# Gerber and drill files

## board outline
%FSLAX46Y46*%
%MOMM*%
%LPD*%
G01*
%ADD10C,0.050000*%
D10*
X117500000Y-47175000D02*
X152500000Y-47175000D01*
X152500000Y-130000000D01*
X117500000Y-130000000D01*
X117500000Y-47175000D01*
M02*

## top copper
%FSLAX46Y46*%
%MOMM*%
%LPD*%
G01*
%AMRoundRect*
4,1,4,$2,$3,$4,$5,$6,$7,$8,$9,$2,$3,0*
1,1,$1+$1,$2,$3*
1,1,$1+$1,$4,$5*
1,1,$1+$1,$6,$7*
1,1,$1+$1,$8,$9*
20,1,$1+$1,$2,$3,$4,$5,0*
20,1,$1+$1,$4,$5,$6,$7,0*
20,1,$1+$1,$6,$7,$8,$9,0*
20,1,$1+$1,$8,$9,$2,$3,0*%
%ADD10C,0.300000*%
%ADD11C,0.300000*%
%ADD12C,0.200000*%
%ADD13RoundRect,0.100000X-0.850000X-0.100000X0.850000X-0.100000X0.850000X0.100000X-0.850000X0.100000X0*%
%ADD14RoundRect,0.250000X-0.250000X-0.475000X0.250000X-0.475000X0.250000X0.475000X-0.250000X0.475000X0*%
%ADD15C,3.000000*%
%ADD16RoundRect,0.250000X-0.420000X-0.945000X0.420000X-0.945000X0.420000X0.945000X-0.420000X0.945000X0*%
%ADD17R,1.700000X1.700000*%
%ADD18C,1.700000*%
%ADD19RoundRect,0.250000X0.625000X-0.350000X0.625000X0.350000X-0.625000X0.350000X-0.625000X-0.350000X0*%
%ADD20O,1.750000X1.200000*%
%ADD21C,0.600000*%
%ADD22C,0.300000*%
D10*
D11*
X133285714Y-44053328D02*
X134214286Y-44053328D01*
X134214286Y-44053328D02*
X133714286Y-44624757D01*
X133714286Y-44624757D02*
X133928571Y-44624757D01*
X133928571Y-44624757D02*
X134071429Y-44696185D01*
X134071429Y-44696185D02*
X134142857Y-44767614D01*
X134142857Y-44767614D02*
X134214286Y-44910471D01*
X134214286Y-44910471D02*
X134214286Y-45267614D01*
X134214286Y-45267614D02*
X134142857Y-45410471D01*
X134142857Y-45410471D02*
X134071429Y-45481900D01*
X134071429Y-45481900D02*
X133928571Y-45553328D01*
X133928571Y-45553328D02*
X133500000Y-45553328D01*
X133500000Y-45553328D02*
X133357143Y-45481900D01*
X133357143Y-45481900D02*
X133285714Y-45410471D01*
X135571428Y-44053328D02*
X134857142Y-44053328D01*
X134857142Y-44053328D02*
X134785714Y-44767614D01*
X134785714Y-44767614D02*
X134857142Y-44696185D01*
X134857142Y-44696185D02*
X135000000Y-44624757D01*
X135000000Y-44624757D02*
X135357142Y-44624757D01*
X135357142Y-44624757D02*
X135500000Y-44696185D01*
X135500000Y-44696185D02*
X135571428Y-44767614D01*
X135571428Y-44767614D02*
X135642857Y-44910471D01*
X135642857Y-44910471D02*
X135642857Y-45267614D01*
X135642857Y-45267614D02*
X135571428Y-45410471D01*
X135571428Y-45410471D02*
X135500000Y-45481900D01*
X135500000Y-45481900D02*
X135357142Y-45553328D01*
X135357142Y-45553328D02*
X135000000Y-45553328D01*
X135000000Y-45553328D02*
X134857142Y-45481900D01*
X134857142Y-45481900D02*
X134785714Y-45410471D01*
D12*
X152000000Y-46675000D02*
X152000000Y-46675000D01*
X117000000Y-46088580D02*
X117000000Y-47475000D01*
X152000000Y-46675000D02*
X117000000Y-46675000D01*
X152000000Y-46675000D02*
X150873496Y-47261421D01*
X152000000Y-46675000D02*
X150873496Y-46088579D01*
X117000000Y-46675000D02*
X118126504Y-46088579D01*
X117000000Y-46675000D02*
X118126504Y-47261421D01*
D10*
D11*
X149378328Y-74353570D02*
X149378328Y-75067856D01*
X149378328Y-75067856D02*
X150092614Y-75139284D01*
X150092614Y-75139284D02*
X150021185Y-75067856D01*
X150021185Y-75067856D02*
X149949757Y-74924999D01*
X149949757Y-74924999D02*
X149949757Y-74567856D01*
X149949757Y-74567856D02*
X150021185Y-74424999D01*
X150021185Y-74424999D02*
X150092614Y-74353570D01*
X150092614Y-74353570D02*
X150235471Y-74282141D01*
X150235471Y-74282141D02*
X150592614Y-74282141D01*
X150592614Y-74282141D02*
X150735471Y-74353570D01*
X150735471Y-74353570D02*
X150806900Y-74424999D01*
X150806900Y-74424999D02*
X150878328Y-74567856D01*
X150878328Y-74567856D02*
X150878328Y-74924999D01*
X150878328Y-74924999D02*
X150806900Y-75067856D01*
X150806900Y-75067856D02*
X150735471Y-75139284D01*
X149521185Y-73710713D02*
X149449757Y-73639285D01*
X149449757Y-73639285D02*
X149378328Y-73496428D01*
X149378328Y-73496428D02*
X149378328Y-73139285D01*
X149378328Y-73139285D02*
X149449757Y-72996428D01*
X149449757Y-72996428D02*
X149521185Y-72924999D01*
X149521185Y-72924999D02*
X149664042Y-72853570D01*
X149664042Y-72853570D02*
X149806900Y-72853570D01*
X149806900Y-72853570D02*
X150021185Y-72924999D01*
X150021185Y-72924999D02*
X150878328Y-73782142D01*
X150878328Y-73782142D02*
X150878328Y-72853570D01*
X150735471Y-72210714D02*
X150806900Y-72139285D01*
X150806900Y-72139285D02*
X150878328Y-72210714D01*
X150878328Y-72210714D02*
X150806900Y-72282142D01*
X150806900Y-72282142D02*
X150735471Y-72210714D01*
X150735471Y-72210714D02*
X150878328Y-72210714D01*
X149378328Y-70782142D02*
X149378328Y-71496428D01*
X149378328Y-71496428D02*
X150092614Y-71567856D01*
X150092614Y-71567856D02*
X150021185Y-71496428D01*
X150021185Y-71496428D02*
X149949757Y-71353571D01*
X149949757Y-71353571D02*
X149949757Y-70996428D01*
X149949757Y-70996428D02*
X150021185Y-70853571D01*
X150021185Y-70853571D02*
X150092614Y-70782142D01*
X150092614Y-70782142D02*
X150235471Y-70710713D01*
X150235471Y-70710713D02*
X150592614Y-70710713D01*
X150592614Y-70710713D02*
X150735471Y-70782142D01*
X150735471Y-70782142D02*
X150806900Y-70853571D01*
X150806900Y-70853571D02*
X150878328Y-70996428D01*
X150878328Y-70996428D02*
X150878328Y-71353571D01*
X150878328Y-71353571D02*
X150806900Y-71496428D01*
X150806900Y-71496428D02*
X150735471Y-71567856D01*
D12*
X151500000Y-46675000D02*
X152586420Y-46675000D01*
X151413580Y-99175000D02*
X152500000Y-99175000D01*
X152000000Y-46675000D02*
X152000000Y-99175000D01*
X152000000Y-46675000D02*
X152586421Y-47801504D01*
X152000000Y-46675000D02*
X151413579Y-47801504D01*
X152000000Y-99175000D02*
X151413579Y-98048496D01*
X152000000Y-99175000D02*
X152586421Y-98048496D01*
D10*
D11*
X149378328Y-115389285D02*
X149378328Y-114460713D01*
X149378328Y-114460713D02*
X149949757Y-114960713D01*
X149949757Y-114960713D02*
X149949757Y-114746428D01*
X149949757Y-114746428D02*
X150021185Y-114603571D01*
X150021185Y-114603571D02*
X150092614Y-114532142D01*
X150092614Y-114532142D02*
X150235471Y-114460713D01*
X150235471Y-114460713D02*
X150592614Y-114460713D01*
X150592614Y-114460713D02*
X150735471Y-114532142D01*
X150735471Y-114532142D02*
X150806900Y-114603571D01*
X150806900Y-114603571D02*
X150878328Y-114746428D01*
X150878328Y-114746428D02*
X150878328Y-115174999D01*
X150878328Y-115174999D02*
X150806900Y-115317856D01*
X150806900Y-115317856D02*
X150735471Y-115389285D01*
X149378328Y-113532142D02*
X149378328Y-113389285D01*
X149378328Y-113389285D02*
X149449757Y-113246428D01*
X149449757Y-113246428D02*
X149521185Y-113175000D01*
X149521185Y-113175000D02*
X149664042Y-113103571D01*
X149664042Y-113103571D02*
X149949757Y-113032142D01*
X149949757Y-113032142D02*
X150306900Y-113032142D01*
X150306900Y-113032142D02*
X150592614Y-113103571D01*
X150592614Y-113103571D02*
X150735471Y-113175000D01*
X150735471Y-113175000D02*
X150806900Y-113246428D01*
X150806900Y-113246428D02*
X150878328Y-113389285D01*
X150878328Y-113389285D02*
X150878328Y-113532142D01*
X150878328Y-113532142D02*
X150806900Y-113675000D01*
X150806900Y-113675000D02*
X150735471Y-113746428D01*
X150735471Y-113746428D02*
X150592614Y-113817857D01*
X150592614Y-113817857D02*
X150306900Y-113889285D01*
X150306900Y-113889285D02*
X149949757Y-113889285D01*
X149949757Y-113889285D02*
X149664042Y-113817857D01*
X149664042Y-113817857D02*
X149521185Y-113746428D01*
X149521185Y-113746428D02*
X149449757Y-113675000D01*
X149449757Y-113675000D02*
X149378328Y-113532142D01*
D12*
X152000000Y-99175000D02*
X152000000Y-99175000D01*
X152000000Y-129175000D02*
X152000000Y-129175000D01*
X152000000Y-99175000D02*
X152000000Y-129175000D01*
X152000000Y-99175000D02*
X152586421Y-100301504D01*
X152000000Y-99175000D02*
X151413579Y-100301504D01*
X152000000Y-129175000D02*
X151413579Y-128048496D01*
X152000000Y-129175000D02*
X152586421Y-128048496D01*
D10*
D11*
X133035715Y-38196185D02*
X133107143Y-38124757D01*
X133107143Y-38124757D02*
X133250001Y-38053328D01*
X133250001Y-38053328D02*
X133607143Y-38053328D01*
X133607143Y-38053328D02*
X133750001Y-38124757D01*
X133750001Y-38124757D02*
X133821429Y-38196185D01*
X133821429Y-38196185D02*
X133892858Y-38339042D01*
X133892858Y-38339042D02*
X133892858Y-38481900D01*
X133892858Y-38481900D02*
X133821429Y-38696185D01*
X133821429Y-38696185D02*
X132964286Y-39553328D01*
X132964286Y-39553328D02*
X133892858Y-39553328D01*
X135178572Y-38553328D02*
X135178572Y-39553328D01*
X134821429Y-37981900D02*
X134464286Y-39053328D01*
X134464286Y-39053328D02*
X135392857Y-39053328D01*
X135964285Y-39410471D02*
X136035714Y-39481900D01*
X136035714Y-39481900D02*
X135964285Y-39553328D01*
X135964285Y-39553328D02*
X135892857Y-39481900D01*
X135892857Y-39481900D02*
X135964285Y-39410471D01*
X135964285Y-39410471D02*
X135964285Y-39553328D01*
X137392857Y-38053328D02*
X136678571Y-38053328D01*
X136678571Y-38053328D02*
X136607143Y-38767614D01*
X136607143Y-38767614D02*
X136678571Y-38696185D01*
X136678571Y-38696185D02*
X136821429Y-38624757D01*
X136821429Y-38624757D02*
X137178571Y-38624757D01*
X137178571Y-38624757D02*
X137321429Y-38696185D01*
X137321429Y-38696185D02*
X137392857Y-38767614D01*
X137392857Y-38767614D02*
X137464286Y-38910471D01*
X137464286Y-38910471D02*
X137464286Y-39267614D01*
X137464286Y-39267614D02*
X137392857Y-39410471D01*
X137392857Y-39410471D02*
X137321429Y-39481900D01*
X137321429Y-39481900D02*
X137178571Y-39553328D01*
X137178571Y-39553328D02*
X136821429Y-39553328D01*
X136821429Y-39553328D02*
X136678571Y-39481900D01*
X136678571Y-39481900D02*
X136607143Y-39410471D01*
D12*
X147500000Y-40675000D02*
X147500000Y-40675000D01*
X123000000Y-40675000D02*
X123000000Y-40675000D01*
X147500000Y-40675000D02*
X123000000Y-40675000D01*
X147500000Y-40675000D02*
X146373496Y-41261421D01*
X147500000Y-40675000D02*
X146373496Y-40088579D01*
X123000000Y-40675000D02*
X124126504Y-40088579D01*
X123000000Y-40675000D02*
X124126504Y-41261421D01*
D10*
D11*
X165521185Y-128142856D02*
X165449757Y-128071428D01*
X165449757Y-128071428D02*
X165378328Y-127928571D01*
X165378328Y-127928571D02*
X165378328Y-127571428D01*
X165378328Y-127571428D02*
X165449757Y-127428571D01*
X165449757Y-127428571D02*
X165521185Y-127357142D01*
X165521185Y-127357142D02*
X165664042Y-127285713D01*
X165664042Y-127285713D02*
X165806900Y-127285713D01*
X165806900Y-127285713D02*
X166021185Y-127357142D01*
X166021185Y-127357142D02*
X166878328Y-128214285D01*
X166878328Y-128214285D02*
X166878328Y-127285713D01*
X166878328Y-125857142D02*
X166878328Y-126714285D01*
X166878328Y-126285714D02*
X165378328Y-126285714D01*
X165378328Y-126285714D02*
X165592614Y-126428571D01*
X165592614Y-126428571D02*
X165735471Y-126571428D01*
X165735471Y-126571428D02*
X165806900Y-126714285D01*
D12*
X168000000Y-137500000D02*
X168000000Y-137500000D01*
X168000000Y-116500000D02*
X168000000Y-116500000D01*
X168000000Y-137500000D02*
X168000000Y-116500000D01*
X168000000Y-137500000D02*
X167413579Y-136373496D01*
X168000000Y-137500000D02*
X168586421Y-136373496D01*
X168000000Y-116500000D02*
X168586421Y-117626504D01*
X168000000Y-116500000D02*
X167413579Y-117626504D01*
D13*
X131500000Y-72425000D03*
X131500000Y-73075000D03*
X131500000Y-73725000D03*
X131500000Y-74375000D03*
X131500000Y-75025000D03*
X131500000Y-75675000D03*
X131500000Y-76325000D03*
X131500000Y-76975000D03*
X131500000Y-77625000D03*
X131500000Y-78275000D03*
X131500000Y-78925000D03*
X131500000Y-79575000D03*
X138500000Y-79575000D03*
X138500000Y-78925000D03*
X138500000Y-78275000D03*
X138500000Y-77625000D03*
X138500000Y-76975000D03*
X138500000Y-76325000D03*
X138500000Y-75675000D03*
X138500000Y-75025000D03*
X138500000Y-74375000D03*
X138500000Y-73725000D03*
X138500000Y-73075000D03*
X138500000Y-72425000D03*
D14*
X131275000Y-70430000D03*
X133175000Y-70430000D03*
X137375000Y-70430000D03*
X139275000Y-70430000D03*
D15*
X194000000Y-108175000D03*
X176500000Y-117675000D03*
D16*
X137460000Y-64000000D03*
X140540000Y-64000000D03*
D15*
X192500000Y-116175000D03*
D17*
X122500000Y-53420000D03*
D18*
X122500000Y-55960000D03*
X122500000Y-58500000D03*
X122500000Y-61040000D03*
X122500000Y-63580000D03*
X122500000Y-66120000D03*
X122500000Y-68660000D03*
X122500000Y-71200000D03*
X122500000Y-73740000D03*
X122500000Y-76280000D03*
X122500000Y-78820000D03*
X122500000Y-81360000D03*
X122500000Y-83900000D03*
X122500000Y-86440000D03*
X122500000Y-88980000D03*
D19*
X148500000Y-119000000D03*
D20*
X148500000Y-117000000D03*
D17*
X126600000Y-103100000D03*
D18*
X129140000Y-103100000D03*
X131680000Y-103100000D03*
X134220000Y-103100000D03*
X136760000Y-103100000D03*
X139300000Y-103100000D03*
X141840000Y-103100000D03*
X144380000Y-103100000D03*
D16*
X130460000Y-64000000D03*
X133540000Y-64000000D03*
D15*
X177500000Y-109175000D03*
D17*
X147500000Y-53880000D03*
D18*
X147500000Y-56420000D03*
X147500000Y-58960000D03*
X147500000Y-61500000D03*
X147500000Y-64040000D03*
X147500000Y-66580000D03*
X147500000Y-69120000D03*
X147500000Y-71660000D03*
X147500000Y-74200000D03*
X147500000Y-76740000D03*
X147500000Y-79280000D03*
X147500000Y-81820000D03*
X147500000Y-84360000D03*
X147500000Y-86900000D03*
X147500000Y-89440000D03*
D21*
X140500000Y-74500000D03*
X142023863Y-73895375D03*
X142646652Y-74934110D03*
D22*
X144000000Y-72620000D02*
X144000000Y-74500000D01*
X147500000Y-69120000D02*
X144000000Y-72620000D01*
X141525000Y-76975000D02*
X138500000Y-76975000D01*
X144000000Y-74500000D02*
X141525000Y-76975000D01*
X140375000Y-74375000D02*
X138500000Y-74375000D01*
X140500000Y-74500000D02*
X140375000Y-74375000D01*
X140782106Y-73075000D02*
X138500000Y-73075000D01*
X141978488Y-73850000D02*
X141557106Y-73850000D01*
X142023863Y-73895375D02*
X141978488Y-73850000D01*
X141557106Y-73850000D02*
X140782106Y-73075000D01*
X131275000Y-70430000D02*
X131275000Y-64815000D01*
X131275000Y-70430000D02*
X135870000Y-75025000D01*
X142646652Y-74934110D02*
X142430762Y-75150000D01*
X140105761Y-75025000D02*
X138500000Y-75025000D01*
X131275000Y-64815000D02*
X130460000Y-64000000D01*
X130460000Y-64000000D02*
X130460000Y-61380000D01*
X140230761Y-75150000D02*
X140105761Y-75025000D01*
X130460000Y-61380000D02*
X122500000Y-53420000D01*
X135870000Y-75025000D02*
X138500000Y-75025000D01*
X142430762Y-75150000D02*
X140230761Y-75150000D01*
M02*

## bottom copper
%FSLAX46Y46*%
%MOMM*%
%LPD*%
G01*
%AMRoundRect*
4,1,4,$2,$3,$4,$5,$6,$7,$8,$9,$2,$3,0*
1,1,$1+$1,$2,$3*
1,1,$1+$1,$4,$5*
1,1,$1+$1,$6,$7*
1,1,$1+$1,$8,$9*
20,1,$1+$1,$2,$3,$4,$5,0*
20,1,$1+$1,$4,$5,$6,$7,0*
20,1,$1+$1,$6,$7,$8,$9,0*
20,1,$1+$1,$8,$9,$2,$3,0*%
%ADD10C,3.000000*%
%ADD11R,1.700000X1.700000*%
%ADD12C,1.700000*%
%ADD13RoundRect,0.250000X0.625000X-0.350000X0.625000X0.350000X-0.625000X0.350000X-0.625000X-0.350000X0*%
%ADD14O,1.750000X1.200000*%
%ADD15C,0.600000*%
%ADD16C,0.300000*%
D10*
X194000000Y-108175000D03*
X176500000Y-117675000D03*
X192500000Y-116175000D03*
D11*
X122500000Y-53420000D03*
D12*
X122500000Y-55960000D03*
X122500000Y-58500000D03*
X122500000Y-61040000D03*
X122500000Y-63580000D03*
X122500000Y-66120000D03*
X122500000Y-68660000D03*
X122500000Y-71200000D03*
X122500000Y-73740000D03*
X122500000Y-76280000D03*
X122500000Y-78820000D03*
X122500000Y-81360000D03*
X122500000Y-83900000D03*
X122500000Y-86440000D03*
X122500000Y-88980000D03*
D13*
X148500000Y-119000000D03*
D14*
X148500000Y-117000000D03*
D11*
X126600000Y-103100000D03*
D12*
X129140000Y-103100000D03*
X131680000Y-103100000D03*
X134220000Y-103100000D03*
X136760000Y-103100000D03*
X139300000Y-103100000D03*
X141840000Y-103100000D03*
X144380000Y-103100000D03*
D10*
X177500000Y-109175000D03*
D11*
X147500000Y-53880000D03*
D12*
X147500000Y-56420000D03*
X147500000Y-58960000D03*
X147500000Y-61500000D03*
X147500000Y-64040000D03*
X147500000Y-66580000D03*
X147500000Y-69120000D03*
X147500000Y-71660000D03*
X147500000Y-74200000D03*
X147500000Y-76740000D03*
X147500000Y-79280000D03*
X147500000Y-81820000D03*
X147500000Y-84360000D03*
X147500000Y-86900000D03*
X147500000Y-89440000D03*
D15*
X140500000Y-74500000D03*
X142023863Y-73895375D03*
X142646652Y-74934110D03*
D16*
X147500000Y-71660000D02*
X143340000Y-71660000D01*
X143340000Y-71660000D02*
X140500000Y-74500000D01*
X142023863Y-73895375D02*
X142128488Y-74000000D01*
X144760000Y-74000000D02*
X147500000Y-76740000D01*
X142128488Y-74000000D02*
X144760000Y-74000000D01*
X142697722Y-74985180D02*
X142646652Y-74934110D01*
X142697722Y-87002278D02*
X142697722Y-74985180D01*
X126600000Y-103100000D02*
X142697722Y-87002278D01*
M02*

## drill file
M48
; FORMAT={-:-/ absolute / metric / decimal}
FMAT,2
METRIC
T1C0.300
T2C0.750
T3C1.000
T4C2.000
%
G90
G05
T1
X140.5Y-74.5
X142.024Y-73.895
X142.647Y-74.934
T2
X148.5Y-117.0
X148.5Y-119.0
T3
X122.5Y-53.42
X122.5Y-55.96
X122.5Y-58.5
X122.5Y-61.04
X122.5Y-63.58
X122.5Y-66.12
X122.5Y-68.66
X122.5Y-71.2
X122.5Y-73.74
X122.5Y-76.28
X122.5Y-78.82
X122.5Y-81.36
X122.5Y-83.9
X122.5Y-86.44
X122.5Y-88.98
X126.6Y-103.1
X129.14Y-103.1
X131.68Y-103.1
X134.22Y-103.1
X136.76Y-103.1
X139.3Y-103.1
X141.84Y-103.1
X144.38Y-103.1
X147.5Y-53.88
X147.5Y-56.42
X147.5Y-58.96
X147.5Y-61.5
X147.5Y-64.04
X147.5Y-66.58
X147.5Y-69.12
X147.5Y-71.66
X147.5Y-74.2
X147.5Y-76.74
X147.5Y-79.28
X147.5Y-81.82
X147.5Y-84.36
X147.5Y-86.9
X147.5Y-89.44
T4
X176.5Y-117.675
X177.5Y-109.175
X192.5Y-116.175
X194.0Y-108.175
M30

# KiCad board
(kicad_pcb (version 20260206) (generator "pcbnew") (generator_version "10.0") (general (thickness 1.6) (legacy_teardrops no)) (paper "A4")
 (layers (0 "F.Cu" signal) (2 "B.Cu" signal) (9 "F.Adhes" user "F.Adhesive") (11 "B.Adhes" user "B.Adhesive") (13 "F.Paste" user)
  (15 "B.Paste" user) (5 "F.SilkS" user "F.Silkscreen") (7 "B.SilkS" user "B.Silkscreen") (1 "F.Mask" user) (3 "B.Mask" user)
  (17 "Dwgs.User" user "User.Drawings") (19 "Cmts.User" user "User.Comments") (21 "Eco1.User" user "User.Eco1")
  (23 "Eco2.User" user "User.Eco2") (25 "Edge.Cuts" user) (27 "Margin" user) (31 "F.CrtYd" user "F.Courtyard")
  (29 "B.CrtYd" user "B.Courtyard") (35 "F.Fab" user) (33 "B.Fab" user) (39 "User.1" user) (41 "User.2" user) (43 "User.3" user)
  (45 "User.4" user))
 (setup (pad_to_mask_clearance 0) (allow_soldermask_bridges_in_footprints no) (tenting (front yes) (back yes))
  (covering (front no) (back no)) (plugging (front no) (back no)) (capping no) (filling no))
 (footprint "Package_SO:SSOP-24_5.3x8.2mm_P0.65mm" (layer "F.Cu") (at 135 76)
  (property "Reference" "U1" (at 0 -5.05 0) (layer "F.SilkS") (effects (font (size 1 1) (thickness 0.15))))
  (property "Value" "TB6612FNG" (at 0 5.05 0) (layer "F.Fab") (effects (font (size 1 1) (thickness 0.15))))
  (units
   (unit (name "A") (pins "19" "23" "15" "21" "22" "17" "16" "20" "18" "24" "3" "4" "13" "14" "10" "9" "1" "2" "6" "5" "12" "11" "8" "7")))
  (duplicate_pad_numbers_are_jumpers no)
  (pad "1" smd roundrect (at -3.5 -3.575) (size 1.9 0.4) (layers "F.Cu" "F.Mask" "F.Paste") (roundrect_rratio 0.25) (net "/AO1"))
  (pad "2" smd roundrect (at -3.5 -2.925) (size 1.9 0.4) (layers "F.Cu" "F.Mask" "F.Paste") (roundrect_rratio 0.25) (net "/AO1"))
  (pad "3" smd roundrect (at -3.5 -2.275) (size 1.9 0.4) (layers "F.Cu" "F.Mask" "F.Paste") (roundrect_rratio 0.25) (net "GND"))
  (pad "4" smd roundrect (at -3.5 -1.625) (size 1.9 0.4) (layers "F.Cu" "F.Mask" "F.Paste") (roundrect_rratio 0.25) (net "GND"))
  (pad "5" smd roundrect (at -3.5 -0.975) (size 1.9 0.4) (layers "F.Cu" "F.Mask" "F.Paste") (roundrect_rratio 0.25) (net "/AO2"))
  (pad "6" smd roundrect (at -3.5 -0.325) (size 1.9 0.4) (layers "F.Cu" "F.Mask" "F.Paste") (roundrect_rratio 0.25) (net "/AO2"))
  (pad "7" smd roundrect (at -3.5 0.325) (size 1.9 0.4) (layers "F.Cu" "F.Mask" "F.Paste") (roundrect_rratio 0.25) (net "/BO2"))
  (pad "8" smd roundrect (at -3.5 0.975) (size 1.9 0.4) (layers "F.Cu" "F.Mask" "F.Paste") (roundrect_rratio 0.25) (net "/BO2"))
  (pad "9" smd roundrect (at -3.5 1.625) (size 1.9 0.4) (layers "F.Cu" "F.Mask" "F.Paste") (roundrect_rratio 0.25) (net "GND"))
  (pad "10" smd roundrect (at -3.5 2.275) (size 1.9 0.4) (layers "F.Cu" "F.Mask" "F.Paste") (roundrect_rratio 0.25) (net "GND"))
  (pad "11" smd roundrect (at -3.5 2.925) (size 1.9 0.4) (layers "F.Cu" "F.Mask" "F.Paste") (roundrect_rratio 0.25) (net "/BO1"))
  (pad "12" smd roundrect (at -3.5 3.575) (size 1.9 0.4) (layers "F.Cu" "F.Mask" "F.Paste") (roundrect_rratio 0.25) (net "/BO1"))
  (pad "13" smd roundrect (at 3.5 3.575) (size 1.9 0.4) (layers "F.Cu" "F.Mask" "F.Paste") (roundrect_rratio 0.25) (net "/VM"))
  (pad "14" smd roundrect (at 3.5 2.925) (size 1.9 0.4) (layers "F.Cu" "F.Mask" "F.Paste") (roundrect_rratio 0.25) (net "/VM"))
  (pad "15" smd roundrect (at 3.5 2.275) (size 1.9 0.4) (layers "F.Cu" "F.Mask" "F.Paste") (roundrect_rratio 0.25) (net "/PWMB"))
  (pad "16" smd roundrect (at 3.5 1.625) (size 1.9 0.4) (layers "F.Cu" "F.Mask" "F.Paste") (roundrect_rratio 0.25) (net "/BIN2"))
  (pad "17" smd roundrect (at 3.5 0.975) (size 1.9 0.4) (layers "F.Cu" "F.Mask" "F.Paste") (roundrect_rratio 0.25) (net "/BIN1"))
  (pad "18" smd roundrect (at 3.5 0.325) (size 1.9 0.4) (layers "F.Cu" "F.Mask" "F.Paste") (roundrect_rratio 0.25) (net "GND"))
  (pad "19" smd roundrect (at 3.5 -0.325) (size 1.9 0.4) (layers "F.Cu" "F.Mask" "F.Paste") (roundrect_rratio 0.25) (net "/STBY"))
  (pad "20" smd roundrect (at 3.5 -0.975) (size 1.9 0.4) (layers "F.Cu" "F.Mask" "F.Paste") (roundrect_rratio 0.25) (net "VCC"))
  (pad "21" smd roundrect (at 3.5 -1.625) (size 1.9 0.4) (layers "F.Cu" "F.Mask" "F.Paste") (roundrect_rratio 0.25) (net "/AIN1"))
  (pad "22" smd roundrect (at 3.5 -2.275) (size 1.9 0.4) (layers "F.Cu" "F.Mask" "F.Paste") (roundrect_rratio 0.25) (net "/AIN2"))
  (pad "23" smd roundrect (at 3.5 -2.925) (size 1.9 0.4) (layers "F.Cu" "F.Mask" "F.Paste") (roundrect_rratio 0.25) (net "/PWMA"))
  (pad "24" smd roundrect (at 3.5 -3.575) (size 1.9 0.4) (layers "F.Cu" "F.Mask" "F.Paste") (roundrect_rratio 0.25) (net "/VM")))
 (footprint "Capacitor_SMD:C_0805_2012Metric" (layer "F.Cu") (at 132.225 70.43)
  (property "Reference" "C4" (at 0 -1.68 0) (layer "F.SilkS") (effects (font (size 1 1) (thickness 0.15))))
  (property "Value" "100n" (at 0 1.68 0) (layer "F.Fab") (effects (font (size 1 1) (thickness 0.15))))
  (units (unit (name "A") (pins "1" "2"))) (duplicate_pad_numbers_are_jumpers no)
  (pad "1" smd roundrect (at -0.95 0) (size 1 1.45) (layers "F.Cu" "F.Mask" "F.Paste") (roundrect_rratio 0.25) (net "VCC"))
  (pad "2" smd roundrect (at 0.95 0) (size 1 1.45) (layers "F.Cu" "F.Mask" "F.Paste") (roundrect_rratio 0.25) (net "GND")))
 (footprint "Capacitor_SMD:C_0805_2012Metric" (layer "F.Cu") (at 138.325 70.43)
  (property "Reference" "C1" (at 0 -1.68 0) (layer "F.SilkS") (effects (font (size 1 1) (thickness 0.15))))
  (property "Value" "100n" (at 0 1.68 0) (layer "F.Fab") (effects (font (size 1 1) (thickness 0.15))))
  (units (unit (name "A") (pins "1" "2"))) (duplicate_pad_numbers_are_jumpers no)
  (pad "1" smd roundrect (at -0.95 0) (size 1 1.45) (layers "F.Cu" "F.Mask" "F.Paste") (roundrect_rratio 0.25) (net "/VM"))
  (pad "2" smd roundrect (at 0.95 0) (size 1 1.45) (layers "F.Cu" "F.Mask" "F.Paste") (roundrect_rratio 0.25) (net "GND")))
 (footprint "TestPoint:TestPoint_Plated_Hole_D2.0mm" (layer "F.Cu") (at 194 108.175)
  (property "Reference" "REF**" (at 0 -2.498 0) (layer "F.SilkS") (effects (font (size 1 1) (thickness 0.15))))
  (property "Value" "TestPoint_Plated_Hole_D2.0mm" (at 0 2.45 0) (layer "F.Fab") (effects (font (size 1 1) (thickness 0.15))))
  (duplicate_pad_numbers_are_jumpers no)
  (pad "1" thru_hole circle (at 0 0) (size 3 3) (drill 2) (layers "*.Cu" "*.Mask") (remove_unused_layers no)))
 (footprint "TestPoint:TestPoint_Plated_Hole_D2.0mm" (layer "F.Cu") (at 176.5 117.675)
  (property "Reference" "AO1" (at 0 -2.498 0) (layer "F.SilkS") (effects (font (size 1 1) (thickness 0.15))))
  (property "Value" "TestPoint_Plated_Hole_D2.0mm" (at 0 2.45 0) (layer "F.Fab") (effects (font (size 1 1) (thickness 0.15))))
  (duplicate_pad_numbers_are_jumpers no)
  (pad "1" thru_hole circle (at 0 0) (size 3 3) (drill 2) (layers "*.Cu" "*.Mask") (remove_unused_layers no) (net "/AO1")))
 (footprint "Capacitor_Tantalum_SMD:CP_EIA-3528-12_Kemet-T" (layer "F.Cu") (at 139 64)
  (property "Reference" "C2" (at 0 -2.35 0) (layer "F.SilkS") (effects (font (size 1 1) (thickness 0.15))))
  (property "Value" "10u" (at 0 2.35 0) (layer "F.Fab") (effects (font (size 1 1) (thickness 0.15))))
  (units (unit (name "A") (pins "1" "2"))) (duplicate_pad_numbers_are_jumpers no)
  (pad "1" smd roundrect (at -1.54 0) (size 1.34 2.39) (layers "F.Cu" "F.Mask" "F.Paste") (roundrect_rratio 0.186567) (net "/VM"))
  (pad "2" smd roundrect (at 1.54 0) (size 1.34 2.39) (layers "F.Cu" "F.Mask" "F.Paste") (roundrect_rratio 0.186567) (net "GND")))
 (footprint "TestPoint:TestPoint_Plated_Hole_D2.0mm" (layer "F.Cu") (at 192.5 116.175)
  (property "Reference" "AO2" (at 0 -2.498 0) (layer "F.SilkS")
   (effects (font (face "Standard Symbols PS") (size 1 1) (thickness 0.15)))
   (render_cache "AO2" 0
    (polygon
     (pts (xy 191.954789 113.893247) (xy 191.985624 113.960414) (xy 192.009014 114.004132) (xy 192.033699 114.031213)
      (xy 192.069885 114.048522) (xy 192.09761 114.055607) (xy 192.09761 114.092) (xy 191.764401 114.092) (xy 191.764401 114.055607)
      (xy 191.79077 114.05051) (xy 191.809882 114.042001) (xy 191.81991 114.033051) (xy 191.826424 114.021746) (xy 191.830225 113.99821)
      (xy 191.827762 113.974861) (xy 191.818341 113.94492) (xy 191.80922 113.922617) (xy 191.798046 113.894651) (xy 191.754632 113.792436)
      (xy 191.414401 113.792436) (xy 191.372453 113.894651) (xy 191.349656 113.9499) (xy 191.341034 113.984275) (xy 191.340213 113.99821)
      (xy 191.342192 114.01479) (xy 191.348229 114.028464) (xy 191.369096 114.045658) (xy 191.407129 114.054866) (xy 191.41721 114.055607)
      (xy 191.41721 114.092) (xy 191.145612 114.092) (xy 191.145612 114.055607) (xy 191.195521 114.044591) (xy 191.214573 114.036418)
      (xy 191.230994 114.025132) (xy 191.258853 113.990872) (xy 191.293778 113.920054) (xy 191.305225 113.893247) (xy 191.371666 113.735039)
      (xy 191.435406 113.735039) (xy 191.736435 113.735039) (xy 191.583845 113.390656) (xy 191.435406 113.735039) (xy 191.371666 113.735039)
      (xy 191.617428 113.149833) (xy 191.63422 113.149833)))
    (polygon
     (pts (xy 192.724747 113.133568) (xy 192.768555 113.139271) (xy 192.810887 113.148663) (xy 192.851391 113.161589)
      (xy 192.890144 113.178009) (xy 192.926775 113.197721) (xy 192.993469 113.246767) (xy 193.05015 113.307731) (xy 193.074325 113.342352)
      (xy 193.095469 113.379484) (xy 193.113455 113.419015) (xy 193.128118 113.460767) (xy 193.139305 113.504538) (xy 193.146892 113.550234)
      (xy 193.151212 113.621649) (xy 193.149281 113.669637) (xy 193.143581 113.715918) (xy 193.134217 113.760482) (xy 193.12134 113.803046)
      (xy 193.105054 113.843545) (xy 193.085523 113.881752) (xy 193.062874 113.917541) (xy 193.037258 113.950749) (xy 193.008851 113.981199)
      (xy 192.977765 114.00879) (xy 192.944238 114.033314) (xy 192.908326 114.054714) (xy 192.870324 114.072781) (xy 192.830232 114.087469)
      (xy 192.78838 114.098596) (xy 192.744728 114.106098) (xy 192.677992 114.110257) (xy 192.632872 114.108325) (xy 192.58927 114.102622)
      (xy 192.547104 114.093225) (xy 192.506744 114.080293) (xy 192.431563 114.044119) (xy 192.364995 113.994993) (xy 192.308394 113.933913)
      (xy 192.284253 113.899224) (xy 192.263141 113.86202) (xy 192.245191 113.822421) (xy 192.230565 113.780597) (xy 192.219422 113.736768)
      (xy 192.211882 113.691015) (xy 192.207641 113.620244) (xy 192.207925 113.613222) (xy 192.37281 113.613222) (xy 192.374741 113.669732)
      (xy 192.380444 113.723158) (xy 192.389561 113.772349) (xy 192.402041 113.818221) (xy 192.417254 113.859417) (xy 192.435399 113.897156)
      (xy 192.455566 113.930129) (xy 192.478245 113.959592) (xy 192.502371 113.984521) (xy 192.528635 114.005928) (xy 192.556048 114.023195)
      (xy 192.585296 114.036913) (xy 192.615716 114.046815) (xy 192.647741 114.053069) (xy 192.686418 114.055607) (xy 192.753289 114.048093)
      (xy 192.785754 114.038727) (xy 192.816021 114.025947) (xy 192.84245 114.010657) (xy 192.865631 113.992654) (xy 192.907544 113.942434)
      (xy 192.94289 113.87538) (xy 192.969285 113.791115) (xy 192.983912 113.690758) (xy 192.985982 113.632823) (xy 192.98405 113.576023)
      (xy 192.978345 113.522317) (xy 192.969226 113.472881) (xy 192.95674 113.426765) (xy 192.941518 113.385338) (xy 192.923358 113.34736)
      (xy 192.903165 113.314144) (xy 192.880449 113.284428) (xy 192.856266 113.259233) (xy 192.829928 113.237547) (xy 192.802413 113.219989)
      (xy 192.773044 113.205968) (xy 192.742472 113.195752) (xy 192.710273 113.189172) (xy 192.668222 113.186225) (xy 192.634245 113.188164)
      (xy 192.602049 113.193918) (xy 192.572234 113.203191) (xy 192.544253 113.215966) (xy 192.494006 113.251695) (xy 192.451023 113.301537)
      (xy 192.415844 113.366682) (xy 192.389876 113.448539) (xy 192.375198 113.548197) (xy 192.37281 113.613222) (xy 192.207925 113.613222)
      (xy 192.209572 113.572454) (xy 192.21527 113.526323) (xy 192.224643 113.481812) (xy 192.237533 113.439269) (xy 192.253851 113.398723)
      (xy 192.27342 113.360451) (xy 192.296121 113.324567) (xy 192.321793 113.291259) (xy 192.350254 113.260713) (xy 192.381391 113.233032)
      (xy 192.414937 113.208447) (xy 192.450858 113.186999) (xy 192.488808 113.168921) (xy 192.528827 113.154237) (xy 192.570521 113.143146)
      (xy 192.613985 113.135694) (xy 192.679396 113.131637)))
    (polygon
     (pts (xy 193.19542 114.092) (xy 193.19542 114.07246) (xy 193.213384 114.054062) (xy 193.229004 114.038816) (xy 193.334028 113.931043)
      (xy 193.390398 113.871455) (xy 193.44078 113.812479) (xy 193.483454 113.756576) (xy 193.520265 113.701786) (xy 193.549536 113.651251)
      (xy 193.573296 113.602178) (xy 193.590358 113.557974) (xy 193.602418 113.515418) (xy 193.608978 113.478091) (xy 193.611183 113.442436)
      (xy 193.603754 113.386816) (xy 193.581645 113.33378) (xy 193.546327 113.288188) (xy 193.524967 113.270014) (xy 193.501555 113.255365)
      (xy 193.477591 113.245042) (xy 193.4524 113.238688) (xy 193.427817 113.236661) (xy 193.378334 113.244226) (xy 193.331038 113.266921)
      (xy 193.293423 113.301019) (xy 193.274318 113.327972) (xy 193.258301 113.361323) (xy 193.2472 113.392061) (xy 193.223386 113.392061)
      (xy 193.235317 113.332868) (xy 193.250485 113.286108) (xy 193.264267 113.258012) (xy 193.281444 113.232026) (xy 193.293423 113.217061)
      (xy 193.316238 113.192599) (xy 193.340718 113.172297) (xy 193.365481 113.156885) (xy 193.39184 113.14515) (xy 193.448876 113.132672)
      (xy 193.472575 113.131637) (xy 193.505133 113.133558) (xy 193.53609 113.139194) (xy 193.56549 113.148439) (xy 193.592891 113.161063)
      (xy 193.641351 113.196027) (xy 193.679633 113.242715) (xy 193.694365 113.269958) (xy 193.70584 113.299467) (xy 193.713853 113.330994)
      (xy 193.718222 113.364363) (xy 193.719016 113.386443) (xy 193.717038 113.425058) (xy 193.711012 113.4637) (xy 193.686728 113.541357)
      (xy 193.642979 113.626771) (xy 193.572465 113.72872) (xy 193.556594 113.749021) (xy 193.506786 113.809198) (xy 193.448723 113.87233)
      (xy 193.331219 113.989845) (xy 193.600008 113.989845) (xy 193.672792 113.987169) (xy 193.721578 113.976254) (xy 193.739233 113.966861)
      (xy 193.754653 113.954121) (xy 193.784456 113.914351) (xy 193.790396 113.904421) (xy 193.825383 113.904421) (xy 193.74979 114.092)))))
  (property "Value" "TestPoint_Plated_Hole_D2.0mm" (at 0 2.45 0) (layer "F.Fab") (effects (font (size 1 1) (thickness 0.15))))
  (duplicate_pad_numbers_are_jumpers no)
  (pad "1" thru_hole circle (at 0 0) (size 3 3) (drill 2) (layers "*.Cu" "*.Mask") (remove_unused_layers no) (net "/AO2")))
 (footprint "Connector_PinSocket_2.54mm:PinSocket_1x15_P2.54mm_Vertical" (layer "F.Cu") (at 122.5 53.42)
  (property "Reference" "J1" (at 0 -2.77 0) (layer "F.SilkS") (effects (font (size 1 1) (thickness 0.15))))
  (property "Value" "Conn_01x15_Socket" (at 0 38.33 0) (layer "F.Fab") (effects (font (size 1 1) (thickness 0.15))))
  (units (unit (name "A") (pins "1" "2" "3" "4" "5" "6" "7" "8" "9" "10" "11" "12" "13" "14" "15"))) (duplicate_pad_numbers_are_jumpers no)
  (pad "1" thru_hole rect (at 0 0) (size 1.7 1.7) (drill 1) (layers "*.Cu" "*.Mask") (remove_unused_layers no) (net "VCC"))
  (pad "2" thru_hole circle (at 0 2.54) (size 1.7 1.7) (drill 1) (layers "*.Cu" "*.Mask") (remove_unused_layers no) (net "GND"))
  (pad "3" thru_hole circle (at 0 5.08) (size 1.7 1.7) (drill 1) (layers "*.Cu" "*.Mask") (remove_unused_layers no)
   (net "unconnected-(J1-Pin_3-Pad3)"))
  (pad "4" thru_hole circle (at 0 7.62) (size 1.7 1.7) (drill 1) (layers "*.Cu" "*.Mask") (remove_unused_layers no)
   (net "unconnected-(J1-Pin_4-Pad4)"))
  (pad "5" thru_hole circle (at 0 10.16) (size 1.7 1.7) (drill 1) (layers "*.Cu" "*.Mask") (remove_unused_layers no)
   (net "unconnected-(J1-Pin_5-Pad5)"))
  (pad "6" thru_hole circle (at 0 12.7) (size 1.7 1.7) (drill 1) (layers "*.Cu" "*.Mask") (remove_unused_layers no) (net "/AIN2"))
  (pad "7" thru_hole circle (at 0 15.24) (size 1.7 1.7) (drill 1) (layers "*.Cu" "*.Mask") (remove_unused_layers no) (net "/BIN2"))
  (pad "8" thru_hole circle (at 0 17.78) (size 1.7 1.7) (drill 1) (layers "*.Cu" "*.Mask") (remove_unused_layers no)
   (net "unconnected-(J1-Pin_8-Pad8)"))
  (pad "9" thru_hole circle (at 0 20.32) (size 1.7 1.7) (drill 1) (layers "*.Cu" "*.Mask") (remove_unused_layers no)
   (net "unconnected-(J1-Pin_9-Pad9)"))
  (pad "10" thru_hole circle (at 0 22.86) (size 1.7 1.7) (drill 1) (layers "*.Cu" "*.Mask") (remove_unused_layers no)
   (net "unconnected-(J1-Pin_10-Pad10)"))
  (pad "11" thru_hole circle (at 0 25.4) (size 1.7 1.7) (drill 1) (layers "*.Cu" "*.Mask") (remove_unused_layers no) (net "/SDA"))
  (pad "12" thru_hole circle (at 0 27.94) (size 1.7 1.7) (drill 1) (layers "*.Cu" "*.Mask") (remove_unused_layers no)
   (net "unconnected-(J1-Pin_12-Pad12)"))
  (pad "13" thru_hole circle (at 0 30.48) (size 1.7 1.7) (drill 1) (layers "*.Cu" "*.Mask") (remove_unused_layers no)
   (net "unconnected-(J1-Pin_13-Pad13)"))
  (pad "14" thru_hole circle (at 0 33.02) (size 1.7 1.7) (drill 1) (layers "*.Cu" "*.Mask") (remove_unused_layers no) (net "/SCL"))
  (pad "15" thru_hole circle (at 0 35.56) (size 1.7 1.7) (drill 1) (layers "*.Cu" "*.Mask") (remove_unused_layers no) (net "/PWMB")))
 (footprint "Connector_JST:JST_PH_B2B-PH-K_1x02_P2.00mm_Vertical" (layer "F.Cu") (at 148.5 119 90)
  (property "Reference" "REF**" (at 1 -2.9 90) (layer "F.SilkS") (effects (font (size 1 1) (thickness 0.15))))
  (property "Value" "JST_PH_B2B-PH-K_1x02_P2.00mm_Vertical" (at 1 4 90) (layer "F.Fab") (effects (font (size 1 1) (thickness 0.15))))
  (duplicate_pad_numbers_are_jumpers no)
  (pad "1" thru_hole roundrect (at 0 0 90) (size 1.2 1.75) (drill 0.75) (layers "*.Cu" "*.Mask") (remove_unused_layers no)
   (roundrect_rratio 0.208333) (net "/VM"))
  (pad "2" thru_hole oval (at 2 0 90) (size 1.2 1.75) (drill 0.75) (layers "*.Cu" "*.Mask") (remove_unused_layers no) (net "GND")))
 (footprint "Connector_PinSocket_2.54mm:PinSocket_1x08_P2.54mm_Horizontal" (layer "F.Cu") (at 126.6 103.1 90)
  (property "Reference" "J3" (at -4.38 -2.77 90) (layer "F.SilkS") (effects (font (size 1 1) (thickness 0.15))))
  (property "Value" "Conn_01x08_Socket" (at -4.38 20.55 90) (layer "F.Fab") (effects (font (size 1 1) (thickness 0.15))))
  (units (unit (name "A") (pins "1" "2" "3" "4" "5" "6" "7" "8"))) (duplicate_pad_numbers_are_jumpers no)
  (pad "1" thru_hole rect (at 0 0 90) (size 1.7 1.7) (drill 1) (layers "*.Cu" "*.Mask") (remove_unused_layers no) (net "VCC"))
  (pad "2" thru_hole circle (at 0 2.54 90) (size 1.7 1.7) (drill 1) (layers "*.Cu" "*.Mask") (remove_unused_layers no) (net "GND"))
  (pad "3" thru_hole circle (at 0 5.08 90) (size 1.7 1.7) (drill 1) (layers "*.Cu" "*.Mask") (remove_unused_layers no) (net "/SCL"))
  (pad "4" thru_hole circle (at 0 7.62 90) (size 1.7 1.7) (drill 1) (layers "*.Cu" "*.Mask") (remove_unused_layers no) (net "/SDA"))
  (pad "5" thru_hole circle (at 0 10.16 90) (size 1.7 1.7) (drill 1) (layers "*.Cu" "*.Mask") (remove_unused_layers no) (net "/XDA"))
  (pad "6" thru_hole circle (at 0 12.7 90) (size 1.7 1.7) (drill 1) (layers "*.Cu" "*.Mask") (remove_unused_layers no) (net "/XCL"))
  (pad "7" thru_hole circle (at 0 15.24 90) (size 1.7 1.7) (drill 1) (layers "*.Cu" "*.Mask") (remove_unused_layers no) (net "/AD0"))
  (pad "8" thru_hole circle (at 0 17.78 90) (size 1.7 1.7) (drill 1) (layers "*.Cu" "*.Mask") (remove_unused_layers no) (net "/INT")))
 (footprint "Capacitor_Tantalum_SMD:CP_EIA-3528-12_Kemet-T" (layer "F.Cu") (at 132 64)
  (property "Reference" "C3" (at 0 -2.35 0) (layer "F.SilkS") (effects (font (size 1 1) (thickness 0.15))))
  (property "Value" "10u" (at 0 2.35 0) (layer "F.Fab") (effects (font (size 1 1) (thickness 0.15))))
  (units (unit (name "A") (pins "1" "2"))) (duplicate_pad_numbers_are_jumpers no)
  (pad "1" smd roundrect (at -1.54 0) (size 1.34 2.39) (layers "F.Cu" "F.Mask" "F.Paste") (roundrect_rratio 0.186567) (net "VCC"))
  (pad "2" smd roundrect (at 1.54 0) (size 1.34 2.39) (layers "F.Cu" "F.Mask" "F.Paste") (roundrect_rratio 0.186567) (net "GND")))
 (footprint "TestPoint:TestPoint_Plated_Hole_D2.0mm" (layer "F.Cu") (at 177.5 109.175)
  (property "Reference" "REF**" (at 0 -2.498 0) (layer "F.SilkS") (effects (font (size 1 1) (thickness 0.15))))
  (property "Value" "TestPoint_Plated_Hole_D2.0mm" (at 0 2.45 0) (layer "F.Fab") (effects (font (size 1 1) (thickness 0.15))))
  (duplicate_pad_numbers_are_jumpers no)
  (pad "1" thru_hole circle (at 0 0) (size 3 3) (drill 2) (layers "*.Cu" "*.Mask") (remove_unused_layers no)))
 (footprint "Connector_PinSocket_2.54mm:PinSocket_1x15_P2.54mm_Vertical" (layer "F.Cu") (at 147.5 53.88)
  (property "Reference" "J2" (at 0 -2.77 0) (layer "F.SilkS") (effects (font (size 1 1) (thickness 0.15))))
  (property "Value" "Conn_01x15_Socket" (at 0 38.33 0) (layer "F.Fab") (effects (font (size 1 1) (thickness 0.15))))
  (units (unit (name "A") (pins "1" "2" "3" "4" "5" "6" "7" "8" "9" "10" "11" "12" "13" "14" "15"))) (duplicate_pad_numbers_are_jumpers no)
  (pad "1" thru_hole rect (at 0 0) (size 1.7 1.7) (drill 1) (layers "*.Cu" "*.Mask") (remove_unused_layers no)
   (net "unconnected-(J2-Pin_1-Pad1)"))
  (pad "2" thru_hole circle (at 0 2.54) (size 1.7 1.7) (drill 1) (layers "*.Cu" "*.Mask") (remove_unused_layers no)
   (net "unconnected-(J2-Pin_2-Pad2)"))
  (pad "3" thru_hole circle (at 0 5.08) (size 1.7 1.7) (drill 1) (layers "*.Cu" "*.Mask") (remove_unused_layers no)
   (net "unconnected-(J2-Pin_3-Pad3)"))
  (pad "4" thru_hole circle (at 0 7.62) (size 1.7 1.7) (drill 1) (layers "*.Cu" "*.Mask") (remove_unused_layers no)
   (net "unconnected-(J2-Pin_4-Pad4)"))
  (pad "5" thru_hole circle (at 0 10.16) (size 1.7 1.7) (drill 1) (layers "*.Cu" "*.Mask") (remove_unused_layers no)
   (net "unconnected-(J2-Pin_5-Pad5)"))
  (pad "6" thru_hole circle (at 0 12.7) (size 1.7 1.7) (drill 1) (layers "*.Cu" "*.Mask") (remove_unused_layers no)
   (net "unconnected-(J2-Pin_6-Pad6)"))
  (pad "7" thru_hole circle (at 0 15.24) (size 1.7 1.7) (drill 1) (layers "*.Cu" "*.Mask") (remove_unused_layers no) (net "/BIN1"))
  (pad "8" thru_hole circle (at 0 17.78) (size 1.7 1.7) (drill 1) (layers "*.Cu" "*.Mask") (remove_unused_layers no) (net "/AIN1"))
  (pad "9" thru_hole circle (at 0 20.32) (size 1.7 1.7) (drill 1) (layers "*.Cu" "*.Mask") (remove_unused_layers no)
   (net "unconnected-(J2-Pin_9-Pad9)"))
  (pad "10" thru_hole circle (at 0 22.86) (size 1.7 1.7) (drill 1) (layers "*.Cu" "*.Mask") (remove_unused_layers no) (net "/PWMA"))
  (pad "11" thru_hole circle (at 0 25.4) (size 1.7 1.7) (drill 1) (layers "*.Cu" "*.Mask") (remove_unused_layers no)
   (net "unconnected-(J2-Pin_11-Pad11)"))
  (pad "12" thru_hole circle (at 0 27.94) (size 1.7 1.7) (drill 1) (layers "*.Cu" "*.Mask") (remove_unused_layers no)
   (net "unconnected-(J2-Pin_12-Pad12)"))
  (pad "13" thru_hole circle (at 0 30.48) (size 1.7 1.7) (drill 1) (layers "*.Cu" "*.Mask") (remove_unused_layers no)
   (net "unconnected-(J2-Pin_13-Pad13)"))
  (pad "14" thru_hole circle (at 0 33.02) (size 1.7 1.7) (drill 1) (layers "*.Cu" "*.Mask") (remove_unused_layers no)
   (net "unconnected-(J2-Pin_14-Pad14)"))
  (pad "15" thru_hole circle (at 0 35.56) (size 1.7 1.7) (drill 1) (layers "*.Cu" "*.Mask") (remove_unused_layers no)
   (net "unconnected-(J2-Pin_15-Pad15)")))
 (gr_rect (start 117.5 47.175) (end 152.5 130) (stroke (width 0.05) (type default)) (fill no) (layer "Edge.Cuts"))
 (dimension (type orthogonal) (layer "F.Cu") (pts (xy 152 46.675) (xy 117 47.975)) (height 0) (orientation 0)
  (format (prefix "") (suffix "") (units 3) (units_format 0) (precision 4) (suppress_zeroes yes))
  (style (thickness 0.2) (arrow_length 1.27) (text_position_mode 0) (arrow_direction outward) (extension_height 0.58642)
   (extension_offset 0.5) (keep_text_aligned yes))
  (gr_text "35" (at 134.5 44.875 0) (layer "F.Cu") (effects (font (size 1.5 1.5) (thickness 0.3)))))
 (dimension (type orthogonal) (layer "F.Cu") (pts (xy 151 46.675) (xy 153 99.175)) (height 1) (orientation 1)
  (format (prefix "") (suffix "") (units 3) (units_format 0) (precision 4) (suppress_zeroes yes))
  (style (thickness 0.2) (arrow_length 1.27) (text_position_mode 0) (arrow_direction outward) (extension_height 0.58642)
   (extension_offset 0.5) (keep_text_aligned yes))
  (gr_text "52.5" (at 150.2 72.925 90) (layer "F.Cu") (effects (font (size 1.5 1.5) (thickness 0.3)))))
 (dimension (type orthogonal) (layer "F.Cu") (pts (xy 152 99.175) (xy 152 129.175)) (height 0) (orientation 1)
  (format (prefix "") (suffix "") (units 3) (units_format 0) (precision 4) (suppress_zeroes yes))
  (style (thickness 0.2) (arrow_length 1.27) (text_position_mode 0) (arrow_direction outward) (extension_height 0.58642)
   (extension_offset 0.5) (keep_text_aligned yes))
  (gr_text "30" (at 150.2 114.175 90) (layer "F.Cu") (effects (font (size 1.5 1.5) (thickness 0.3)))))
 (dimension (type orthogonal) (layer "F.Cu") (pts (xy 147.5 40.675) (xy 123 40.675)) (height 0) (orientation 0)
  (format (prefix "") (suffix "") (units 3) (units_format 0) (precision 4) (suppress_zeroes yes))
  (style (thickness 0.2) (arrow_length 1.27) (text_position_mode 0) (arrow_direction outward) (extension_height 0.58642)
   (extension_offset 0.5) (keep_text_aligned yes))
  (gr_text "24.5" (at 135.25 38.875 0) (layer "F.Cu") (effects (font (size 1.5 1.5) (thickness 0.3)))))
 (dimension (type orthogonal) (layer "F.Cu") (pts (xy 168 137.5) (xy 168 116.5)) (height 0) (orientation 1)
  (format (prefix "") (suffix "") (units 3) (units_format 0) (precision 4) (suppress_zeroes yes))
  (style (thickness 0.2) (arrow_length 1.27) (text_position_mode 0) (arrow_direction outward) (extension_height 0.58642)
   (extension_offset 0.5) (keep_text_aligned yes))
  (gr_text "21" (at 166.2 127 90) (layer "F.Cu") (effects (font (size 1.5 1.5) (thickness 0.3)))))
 (segment (start 144 72.62) (end 144 74.5) (width 0.3) (layer "F.Cu") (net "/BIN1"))
 (segment (start 147.5 69.12) (end 144 72.62) (width 0.3) (layer "F.Cu") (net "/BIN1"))
 (segment (start 141.525 76.975) (end 138.5 76.975) (width 0.3) (layer "F.Cu") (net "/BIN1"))
 (segment (start 144 74.5) (end 141.525 76.975) (width 0.3) (layer "F.Cu") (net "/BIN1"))
 (segment (start 140.375 74.375) (end 138.5 74.375) (width 0.3) (layer "F.Cu") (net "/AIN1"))
 (segment (start 140.5 74.5) (end 140.375 74.375) (width 0.3) (layer "F.Cu") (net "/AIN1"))
 (via (at 140.5 74.5) (size 0.6) (drill 0.3) (layers "F.Cu" "B.Cu") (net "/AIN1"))
 (segment (start 147.5 71.66) (end 143.34 71.66) (width 0.3) (layer "B.Cu") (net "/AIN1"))
 (segment (start 143.34 71.66) (end 140.5 74.5) (width 0.3) (layer "B.Cu") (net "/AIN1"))
 (segment (start 140.782106 73.075) (end 138.5 73.075) (width 0.3) (layer "F.Cu") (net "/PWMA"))
 (segment (start 141.978488 73.85) (end 141.557106 73.85) (width 0.3) (layer "F.Cu") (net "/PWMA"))
 (segment (start 142.023863 73.895375) (end 141.978488 73.85) (width 0.3) (layer "F.Cu") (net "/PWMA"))
 (segment (start 141.557106 73.85) (end 140.782106 73.075) (width 0.3) (layer "F.Cu") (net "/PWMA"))
 (via (at 142.023863 73.895375) (size 0.6) (drill 0.3) (layers "F.Cu" "B.Cu") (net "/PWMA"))
 (segment (start 142.023863 73.895375) (end 142.128488 74) (width 0.3) (layer "B.Cu") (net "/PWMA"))
 (segment (start 144.76 74) (end 147.5 76.74) (width 0.3) (layer "B.Cu") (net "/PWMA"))
 (segment (start 142.128488 74) (end 144.76 74) (width 0.3) (layer "B.Cu") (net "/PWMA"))
 (segment (start 131.275 70.43) (end 131.275 64.815) (width 0.3) (layer "F.Cu") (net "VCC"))
 (segment (start 131.275 70.43) (end 135.87 75.025) (width 0.3) (layer "F.Cu") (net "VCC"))
 (segment (start 142.646652 74.93411) (end 142.430762 75.15) (width 0.3) (layer "F.Cu") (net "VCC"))
 (segment (start 140.105761 75.025) (end 138.5 75.025) (width 0.3) (layer "F.Cu") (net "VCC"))
 (segment (start 131.275 64.815) (end 130.46 64) (width 0.3) (layer "F.Cu") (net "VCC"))
 (segment (start 130.46 64) (end 130.46 61.38) (width 0.3) (layer "F.Cu") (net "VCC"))
 (segment (start 140.230761 75.15) (end 140.105761 75.025) (width 0.3) (layer "F.Cu") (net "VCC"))
 (segment (start 130.46 61.38) (end 122.5 53.42) (width 0.3) (layer "F.Cu") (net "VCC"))
 (segment (start 135.87 75.025) (end 138.5 75.025) (width 0.3) (layer "F.Cu") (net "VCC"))
 (segment (start 142.430762 75.15) (end 140.230761 75.15) (width 0.3) (layer "F.Cu") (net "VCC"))
 (via (at 142.646652 74.93411) (size 0.6) (drill 0.3) (layers "F.Cu" "B.Cu") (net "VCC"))
 (segment (start 142.697722 74.98518) (end 142.646652 74.93411) (width 0.3) (layer "B.Cu") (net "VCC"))
 (segment (start 142.697722 87.002278) (end 142.697722 74.98518) (width 0.3) (layer "B.Cu") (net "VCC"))
 (segment (start 126.6 103.1) (end 142.697722 87.002278) (width 0.3) (layer "B.Cu") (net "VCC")))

